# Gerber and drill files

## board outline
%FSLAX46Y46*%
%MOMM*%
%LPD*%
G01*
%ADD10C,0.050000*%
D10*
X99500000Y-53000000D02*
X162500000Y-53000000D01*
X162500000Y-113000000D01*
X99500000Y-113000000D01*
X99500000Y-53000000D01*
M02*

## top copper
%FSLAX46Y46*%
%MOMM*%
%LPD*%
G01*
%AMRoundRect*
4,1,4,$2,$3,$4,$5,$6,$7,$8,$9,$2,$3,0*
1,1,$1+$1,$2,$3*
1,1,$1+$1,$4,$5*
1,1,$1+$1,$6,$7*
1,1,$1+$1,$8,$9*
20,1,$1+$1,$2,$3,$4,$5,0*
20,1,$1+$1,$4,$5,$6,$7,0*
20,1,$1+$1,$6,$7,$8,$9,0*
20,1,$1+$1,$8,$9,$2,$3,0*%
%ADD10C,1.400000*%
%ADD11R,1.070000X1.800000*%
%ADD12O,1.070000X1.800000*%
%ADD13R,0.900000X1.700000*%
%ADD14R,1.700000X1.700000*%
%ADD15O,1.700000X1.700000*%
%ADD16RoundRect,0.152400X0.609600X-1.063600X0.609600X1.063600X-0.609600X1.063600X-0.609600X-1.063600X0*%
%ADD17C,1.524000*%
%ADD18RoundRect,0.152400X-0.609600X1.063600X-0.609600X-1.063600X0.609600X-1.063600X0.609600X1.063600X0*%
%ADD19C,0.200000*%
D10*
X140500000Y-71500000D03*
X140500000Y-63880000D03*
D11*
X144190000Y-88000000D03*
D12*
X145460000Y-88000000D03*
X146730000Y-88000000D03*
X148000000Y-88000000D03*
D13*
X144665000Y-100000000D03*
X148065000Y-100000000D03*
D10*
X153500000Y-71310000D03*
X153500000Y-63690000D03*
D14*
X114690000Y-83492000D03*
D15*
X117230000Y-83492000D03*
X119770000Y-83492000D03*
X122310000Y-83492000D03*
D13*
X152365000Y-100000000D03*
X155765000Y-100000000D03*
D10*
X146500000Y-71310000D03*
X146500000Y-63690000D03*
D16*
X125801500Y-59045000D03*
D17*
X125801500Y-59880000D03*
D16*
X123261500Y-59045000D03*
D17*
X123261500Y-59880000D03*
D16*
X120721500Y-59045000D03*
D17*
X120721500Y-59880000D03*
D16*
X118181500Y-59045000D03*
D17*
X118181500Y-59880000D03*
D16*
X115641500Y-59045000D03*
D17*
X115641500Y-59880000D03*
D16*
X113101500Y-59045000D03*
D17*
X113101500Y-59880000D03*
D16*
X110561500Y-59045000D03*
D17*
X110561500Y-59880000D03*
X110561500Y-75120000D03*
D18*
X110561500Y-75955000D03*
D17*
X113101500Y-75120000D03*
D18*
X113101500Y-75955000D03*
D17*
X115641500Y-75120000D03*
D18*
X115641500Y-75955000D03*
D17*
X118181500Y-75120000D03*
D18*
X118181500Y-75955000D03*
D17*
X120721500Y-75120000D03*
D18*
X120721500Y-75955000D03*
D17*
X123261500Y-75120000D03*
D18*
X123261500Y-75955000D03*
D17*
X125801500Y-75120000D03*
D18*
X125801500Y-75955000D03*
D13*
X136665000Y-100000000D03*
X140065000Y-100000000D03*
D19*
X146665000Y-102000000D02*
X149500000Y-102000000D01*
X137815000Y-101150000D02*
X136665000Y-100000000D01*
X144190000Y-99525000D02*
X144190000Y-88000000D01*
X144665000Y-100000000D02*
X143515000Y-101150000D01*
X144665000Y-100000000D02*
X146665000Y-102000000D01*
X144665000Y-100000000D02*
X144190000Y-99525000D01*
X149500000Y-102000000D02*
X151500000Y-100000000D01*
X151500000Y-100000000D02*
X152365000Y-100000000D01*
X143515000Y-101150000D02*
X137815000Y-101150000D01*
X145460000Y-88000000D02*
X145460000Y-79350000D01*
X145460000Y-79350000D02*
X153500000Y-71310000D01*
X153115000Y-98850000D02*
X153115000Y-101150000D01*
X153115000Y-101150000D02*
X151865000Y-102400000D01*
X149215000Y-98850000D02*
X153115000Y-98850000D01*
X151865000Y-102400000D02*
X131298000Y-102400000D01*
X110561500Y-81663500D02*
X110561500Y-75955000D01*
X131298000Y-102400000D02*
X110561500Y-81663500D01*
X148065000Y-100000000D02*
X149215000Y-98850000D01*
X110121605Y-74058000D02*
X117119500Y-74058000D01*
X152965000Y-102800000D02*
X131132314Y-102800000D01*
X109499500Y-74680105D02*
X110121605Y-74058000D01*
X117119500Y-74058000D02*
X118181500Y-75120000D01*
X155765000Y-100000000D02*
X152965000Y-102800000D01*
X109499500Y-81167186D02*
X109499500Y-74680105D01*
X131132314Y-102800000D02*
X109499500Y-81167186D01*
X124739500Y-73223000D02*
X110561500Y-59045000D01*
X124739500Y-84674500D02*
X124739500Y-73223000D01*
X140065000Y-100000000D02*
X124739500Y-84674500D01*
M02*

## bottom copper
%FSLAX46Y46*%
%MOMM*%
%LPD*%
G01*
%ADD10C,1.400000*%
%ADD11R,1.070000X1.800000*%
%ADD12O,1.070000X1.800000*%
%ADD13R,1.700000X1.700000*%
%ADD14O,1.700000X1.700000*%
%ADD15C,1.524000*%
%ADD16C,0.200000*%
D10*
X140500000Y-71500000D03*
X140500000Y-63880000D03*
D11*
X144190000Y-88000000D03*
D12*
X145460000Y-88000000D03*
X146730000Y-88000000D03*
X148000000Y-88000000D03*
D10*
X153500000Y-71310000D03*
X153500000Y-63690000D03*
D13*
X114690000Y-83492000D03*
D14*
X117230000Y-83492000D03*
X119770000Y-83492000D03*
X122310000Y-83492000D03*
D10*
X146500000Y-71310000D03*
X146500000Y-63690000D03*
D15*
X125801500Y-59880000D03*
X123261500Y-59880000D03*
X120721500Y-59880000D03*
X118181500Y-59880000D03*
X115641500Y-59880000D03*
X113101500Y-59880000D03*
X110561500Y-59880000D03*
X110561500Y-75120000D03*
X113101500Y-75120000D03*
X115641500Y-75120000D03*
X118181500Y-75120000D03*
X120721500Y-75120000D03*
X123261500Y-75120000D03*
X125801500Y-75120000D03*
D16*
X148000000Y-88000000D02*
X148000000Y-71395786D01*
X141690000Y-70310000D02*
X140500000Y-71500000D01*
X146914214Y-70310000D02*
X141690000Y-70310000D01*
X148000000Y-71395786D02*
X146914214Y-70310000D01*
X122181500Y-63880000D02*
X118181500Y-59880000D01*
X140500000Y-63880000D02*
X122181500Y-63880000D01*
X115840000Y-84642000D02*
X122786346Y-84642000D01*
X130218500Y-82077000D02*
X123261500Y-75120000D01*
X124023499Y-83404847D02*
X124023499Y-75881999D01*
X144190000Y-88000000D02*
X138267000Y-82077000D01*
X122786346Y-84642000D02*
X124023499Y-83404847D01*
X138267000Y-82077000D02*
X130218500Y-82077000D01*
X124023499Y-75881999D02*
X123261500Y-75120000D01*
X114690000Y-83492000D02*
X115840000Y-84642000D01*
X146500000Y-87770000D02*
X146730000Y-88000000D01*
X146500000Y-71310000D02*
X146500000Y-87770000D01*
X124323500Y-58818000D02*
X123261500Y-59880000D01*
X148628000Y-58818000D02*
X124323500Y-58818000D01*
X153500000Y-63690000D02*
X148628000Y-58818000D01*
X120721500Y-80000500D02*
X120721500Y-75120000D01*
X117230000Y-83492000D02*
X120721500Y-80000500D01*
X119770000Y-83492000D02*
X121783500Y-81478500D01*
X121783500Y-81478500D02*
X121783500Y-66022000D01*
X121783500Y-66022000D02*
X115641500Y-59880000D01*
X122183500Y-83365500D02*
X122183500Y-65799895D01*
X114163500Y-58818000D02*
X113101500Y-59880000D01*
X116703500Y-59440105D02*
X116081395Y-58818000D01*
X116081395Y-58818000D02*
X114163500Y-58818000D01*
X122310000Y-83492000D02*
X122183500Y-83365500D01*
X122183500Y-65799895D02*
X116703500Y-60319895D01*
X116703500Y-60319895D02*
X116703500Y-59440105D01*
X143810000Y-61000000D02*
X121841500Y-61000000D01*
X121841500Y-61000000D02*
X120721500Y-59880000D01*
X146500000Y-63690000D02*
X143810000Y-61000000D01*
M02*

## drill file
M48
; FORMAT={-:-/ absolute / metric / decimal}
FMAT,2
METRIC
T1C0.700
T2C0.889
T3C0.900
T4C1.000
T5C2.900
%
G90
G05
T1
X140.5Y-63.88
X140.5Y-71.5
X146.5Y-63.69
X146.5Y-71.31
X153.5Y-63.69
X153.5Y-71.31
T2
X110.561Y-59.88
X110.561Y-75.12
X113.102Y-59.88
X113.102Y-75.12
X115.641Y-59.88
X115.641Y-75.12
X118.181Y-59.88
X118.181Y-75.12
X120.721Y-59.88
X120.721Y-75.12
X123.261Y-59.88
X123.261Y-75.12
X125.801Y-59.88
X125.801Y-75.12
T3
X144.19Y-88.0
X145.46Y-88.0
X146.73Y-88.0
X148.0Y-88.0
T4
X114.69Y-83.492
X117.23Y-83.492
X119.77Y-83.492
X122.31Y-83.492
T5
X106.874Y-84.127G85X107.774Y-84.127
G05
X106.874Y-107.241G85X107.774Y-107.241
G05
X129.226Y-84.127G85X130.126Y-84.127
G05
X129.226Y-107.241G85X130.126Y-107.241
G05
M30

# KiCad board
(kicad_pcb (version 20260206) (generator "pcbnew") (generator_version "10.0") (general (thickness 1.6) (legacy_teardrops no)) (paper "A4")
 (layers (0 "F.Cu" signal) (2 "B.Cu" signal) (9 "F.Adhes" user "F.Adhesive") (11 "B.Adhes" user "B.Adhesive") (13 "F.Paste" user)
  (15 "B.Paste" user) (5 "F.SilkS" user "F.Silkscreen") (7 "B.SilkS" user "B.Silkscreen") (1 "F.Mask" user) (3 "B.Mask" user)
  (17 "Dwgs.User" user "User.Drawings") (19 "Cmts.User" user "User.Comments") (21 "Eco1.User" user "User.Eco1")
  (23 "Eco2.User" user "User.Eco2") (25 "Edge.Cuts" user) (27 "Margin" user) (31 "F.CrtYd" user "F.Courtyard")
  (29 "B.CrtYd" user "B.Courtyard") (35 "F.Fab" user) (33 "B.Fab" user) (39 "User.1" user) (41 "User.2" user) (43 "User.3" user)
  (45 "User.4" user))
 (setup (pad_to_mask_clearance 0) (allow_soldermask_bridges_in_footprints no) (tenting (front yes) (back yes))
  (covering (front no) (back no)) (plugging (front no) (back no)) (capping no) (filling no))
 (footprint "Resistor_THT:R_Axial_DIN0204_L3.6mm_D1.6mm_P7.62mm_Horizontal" (layer "F.Cu") (at 140.5 71.5 90)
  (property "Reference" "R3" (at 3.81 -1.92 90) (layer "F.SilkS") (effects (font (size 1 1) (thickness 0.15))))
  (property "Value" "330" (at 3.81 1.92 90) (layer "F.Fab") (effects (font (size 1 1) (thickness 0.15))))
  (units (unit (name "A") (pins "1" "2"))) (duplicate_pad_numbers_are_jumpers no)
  (pad "1" thru_hole circle (at 0 0 90) (size 1.4 1.4) (drill 0.7) (layers "*.Cu" "*.Mask") (remove_unused_layers no) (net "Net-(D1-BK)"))
  (pad "2" thru_hole circle (at 7.62 0 90) (size 1.4 1.4) (drill 0.7) (layers "*.Cu" "*.Mask") (remove_unused_layers no) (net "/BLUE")))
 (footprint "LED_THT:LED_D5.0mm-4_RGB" (layer "F.Cu") (at 144.19 88)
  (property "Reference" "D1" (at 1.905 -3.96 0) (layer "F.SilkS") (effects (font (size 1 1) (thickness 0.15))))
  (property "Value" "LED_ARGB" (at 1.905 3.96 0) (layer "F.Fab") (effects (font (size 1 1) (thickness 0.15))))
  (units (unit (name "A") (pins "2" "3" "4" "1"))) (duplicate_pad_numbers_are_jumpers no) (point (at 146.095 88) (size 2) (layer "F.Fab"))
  (pad "1" thru_hole rect (at 0 0) (size 1.07 1.8) (drill 0.9) (layers "*.Cu" "*.Mask") (remove_unused_layers no) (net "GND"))
  (pad "2" thru_hole oval (at 1.27 0) (size 1.07 1.8) (drill 0.9) (layers "*.Cu" "*.Mask") (remove_unused_layers no) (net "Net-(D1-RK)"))
  (pad "3" thru_hole oval (at 2.54 0) (size 1.07 1.8) (drill 0.9) (layers "*.Cu" "*.Mask") (remove_unused_layers no) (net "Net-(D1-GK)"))
  (pad "4" thru_hole oval (at 3.81 0) (size 1.07 1.8) (drill 0.9) (layers "*.Cu" "*.Mask") (remove_unused_layers no) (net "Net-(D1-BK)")))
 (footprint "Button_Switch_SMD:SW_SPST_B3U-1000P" (layer "F.Cu") (at 146.365 100)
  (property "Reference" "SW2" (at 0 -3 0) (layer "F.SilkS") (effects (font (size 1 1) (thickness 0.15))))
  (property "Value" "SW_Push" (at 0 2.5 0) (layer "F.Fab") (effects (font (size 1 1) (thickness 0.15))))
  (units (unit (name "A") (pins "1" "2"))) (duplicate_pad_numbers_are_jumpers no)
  (pad "1" smd rect (at -1.7 0) (size 0.9 1.7) (layers "F.Cu" "F.Mask" "F.Paste") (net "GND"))
  (pad "2" smd rect (at 1.7 0) (size 0.9 1.7) (layers "F.Cu" "F.Mask" "F.Paste") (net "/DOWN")))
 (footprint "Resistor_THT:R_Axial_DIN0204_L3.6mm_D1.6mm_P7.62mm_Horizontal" (layer "F.Cu") (at 153.5 71.31 90)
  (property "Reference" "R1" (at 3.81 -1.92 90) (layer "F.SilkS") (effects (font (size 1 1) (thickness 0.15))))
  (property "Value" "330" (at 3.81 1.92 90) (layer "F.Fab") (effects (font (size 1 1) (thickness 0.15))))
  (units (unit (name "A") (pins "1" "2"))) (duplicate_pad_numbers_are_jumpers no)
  (pad "1" thru_hole circle (at 0 0 90) (size 1.4 1.4) (drill 0.7) (layers "*.Cu" "*.Mask") (remove_unused_layers no) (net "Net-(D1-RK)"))
  (pad "2" thru_hole circle (at 7.62 0 90) (size 1.4 1.4) (drill 0.7) (layers "*.Cu" "*.Mask") (remove_unused_layers no) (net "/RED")))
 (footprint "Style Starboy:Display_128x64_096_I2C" (layer "F.Cu") (at 118.5 83.492)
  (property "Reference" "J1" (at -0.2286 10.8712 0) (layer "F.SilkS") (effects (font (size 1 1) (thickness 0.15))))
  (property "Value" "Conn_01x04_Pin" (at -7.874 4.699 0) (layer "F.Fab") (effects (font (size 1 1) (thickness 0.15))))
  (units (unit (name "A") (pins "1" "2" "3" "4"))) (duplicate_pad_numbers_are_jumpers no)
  (pad "" np_thru_hole oval (at -11.176 0.635) (size 3.8 2.9) (drill oval 3.8 2.9) (layers "*.Cu" "*.Mask"))
  (pad "" np_thru_hole oval (at -11.176 23.749) (size 3.8 2.9) (drill oval 3.8 2.9) (layers "*.Cu" "*.Mask"))
  (pad "" np_thru_hole oval (at 11.176 0.635) (size 3.8 2.9) (drill oval 3.8 2.9) (layers "*.Cu" "*.Mask"))
  (pad "" np_thru_hole oval (at 11.176 23.749) (size 3.8 2.9) (drill oval 3.8 2.9) (layers "*.Cu" "*.Mask"))
  (pad "1" thru_hole rect (at -3.81 0 90) (size 1.7 1.7) (drill 1) (layers "*.Cu" "*.Mask") (remove_unused_layers no) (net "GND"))
  (pad "2" thru_hole oval (at -1.27 0 90) (size 1.7 1.7) (drill 1) (layers "*.Cu" "*.Mask") (remove_unused_layers no) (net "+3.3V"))
  (pad "3" thru_hole oval (at 1.27 0 90) (size 1.7 1.7) (drill 1) (layers "*.Cu" "*.Mask") (remove_unused_layers no) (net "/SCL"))
  (pad "4" thru_hole oval (at 3.81 0 90) (size 1.7 1.7) (drill 1) (layers "*.Cu" "*.Mask") (remove_unused_layers no) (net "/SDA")))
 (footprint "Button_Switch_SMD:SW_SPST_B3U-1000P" (layer "F.Cu") (at 154.065 100)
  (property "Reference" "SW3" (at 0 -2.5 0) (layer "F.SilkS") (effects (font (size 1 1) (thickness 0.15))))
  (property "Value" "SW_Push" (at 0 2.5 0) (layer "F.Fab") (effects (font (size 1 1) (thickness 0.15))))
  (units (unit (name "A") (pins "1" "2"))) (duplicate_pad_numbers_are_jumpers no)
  (pad "1" smd rect (at -1.7 0) (size 0.9 1.7) (layers "F.Cu" "F.Mask" "F.Paste") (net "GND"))
  (pad "2" smd rect (at 1.7 0) (size 0.9 1.7) (layers "F.Cu" "F.Mask" "F.Paste") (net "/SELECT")))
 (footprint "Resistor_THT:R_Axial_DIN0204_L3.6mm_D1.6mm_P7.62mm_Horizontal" (layer "F.Cu") (at 146.5 71.31 90)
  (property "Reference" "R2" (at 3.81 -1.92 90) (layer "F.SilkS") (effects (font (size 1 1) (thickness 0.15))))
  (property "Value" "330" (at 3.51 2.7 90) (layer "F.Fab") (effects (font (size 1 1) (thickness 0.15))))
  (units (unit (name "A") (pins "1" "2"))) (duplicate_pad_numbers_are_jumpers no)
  (pad "1" thru_hole circle (at 0 0 90) (size 1.4 1.4) (drill 0.7) (layers "*.Cu" "*.Mask") (remove_unused_layers no) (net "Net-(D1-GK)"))
  (pad "2" thru_hole circle (at 7.62 0 90) (size 1.4 1.4) (drill 0.7) (layers "*.Cu" "*.Mask") (remove_unused_layers no) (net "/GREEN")))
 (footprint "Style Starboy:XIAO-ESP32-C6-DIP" (layer "F.Cu") (at 118.1815 67.5)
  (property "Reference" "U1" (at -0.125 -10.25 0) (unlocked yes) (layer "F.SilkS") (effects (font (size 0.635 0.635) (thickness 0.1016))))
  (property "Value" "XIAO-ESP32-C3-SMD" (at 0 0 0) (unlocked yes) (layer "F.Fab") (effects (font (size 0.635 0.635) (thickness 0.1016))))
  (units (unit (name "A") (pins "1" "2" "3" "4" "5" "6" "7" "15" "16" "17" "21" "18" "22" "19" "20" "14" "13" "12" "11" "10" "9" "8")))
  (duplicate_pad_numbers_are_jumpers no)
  (pad "1" smd roundrect (at 7.62 -8.455 90) (size 2.432 1.524) (layers "F.Cu" "F.Mask") (roundrect_rratio 0.1)
   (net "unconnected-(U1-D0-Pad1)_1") (thermal_bridge_angle 45))
  (pad "1" thru_hole circle (at 7.62 -7.62 90) (size 1.524 1.524) (drill 0.889) (layers "*.Cu" "*.Mask") (remove_unused_layers no)
   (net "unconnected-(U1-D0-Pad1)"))
  (pad "2" smd roundrect (at 5.08 -8.455 90) (size 2.432 1.524) (layers "F.Cu" "F.Mask") (roundrect_rratio 0.1) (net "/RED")
   (thermal_bridge_angle 45))
  (pad "2" thru_hole circle (at 5.08 -7.62 90) (size 1.524 1.524) (drill 0.889) (layers "*.Cu" "*.Mask") (remove_unused_layers no)
   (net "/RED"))
  (pad "3" smd roundrect (at 2.54 -8.455 90) (size 2.432 1.524) (layers "F.Cu" "F.Mask") (roundrect_rratio 0.1) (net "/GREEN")
   (thermal_bridge_angle 45))
  (pad "3" thru_hole circle (at 2.54 -7.62 90) (size 1.524 1.524) (drill 0.889) (layers "*.Cu" "*.Mask") (remove_unused_layers no)
   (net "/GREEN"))
  (pad "4" smd roundrect (at 0 -8.455 90) (size 2.432 1.524) (layers "F.Cu" "F.Mask") (roundrect_rratio 0.1) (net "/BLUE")
   (thermal_bridge_angle 45))
  (pad "4" thru_hole circle (at 0 -7.62 90) (size 1.524 1.524) (drill 0.889) (layers "*.Cu" "*.Mask") (remove_unused_layers no)
   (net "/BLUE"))
  (pad "5" smd roundrect (at -2.54 -8.455 90) (size 2.432 1.524) (layers "F.Cu" "F.Mask") (roundrect_rratio 0.1) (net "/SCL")
   (thermal_bridge_angle 45))
  (pad "5" thru_hole circle (at -2.54 -7.62 90) (size 1.524 1.524) (drill 0.889) (layers "*.Cu" "*.Mask") (remove_unused_layers no)
   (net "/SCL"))
  (pad "6" smd roundrect (at -5.08 -8.455 90) (size 2.432 1.524) (layers "F.Cu" "F.Mask") (roundrect_rratio 0.1) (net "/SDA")
   (thermal_bridge_angle 45))
  (pad "6" thru_hole circle (at -5.08 -7.62 90) (size 1.524 1.524) (drill 0.889) (layers "*.Cu" "*.Mask") (remove_unused_layers no)
   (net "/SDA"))
  (pad "7" smd roundrect (at -7.62 -8.455 90) (size 2.432 1.524) (layers "F.Cu" "F.Mask") (roundrect_rratio 0.1) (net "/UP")
   (thermal_bridge_angle 45))
  (pad "7" thru_hole circle (at -7.62 -7.62 90) (size 1.524 1.524) (drill 0.889) (layers "*.Cu" "*.Mask") (remove_unused_layers no)
   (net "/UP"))
  (pad "8" thru_hole circle (at -7.62 7.62 270) (size 1.524 1.524) (drill 0.889) (layers "*.Cu" "*.Mask") (remove_unused_layers no)
   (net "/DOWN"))
  (pad "8" smd roundrect (at -7.62 8.455 270) (size 2.432 1.524) (layers "F.Cu" "F.Mask") (roundrect_rratio 0.1) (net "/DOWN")
   (thermal_bridge_angle 45))
  (pad "9" thru_hole circle (at -5.08 7.62 270) (size 1.524 1.524) (drill 0.889) (layers "*.Cu" "*.Mask") (remove_unused_layers no)
   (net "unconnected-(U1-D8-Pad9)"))
  (pad "9" smd roundrect (at -5.08 8.455 270) (size 2.432 1.524) (layers "F.Cu" "F.Mask") (roundrect_rratio 0.1)
   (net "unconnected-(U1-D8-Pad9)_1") (thermal_bridge_angle 45))
  (pad "10" thru_hole circle (at -2.54 7.62 270) (size 1.524 1.524) (drill 0.889) (layers "*.Cu" "*.Mask") (remove_unused_layers no)
   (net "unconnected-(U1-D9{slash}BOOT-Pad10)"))
  (pad "10" smd roundrect (at -2.54 8.455 270) (size 2.432 1.524) (layers "F.Cu" "F.Mask") (roundrect_rratio 0.1)
   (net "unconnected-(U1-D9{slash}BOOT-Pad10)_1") (thermal_bridge_angle 45))
  (pad "11" thru_hole circle (at 0 7.62 270) (size 1.524 1.524) (drill 0.889) (layers "*.Cu" "*.Mask") (remove_unused_layers no)
   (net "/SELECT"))
  (pad "11" smd roundrect (at 0 8.455 270) (size 2.432 1.524) (layers "F.Cu" "F.Mask") (roundrect_rratio 0.1) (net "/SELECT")
   (thermal_bridge_angle 45))
  (pad "12" thru_hole circle (at 2.54 7.62 270) (size 1.524 1.524) (drill 0.889) (layers "*.Cu" "*.Mask") (remove_unused_layers no)
   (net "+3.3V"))
  (pad "12" smd roundrect (at 2.54 8.455 270) (size 2.432 1.524) (layers "F.Cu" "F.Mask") (roundrect_rratio 0.1) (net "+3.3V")
   (thermal_bridge_angle 45))
  (pad "13" thru_hole circle (at 5.08 7.62 270) (size 1.524 1.524) (drill 0.889) (layers "*.Cu" "*.Mask") (remove_unused_layers no)
   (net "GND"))
  (pad "13" smd roundrect (at 5.08 8.455 270) (size 2.432 1.524) (layers "F.Cu" "F.Mask") (roundrect_rratio 0.1) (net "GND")
   (thermal_bridge_angle 45))
  (pad "14" thru_hole circle (at 7.62 7.62 270) (size 1.524 1.524) (drill 0.889) (layers "*.Cu" "*.Mask") (remove_unused_layers no)
   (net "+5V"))
  (pad "14" smd roundrect (at 7.62 8.455 270) (size 2.432 1.524) (layers "F.Cu" "F.Mask") (roundrect_rratio 0.1) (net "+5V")
   (thermal_bridge_angle 45)))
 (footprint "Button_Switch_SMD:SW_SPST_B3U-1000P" (layer "F.Cu") (at 138.365 100)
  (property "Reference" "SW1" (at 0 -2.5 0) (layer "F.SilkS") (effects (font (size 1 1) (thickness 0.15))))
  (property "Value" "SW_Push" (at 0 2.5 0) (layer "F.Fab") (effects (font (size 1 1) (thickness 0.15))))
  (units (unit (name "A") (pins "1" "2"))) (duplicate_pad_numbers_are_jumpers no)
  (pad "1" smd rect (at -1.7 0) (size 0.9 1.7) (layers "F.Cu" "F.Mask" "F.Paste") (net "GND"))
  (pad "2" smd rect (at 1.7 0) (size 0.9 1.7) (layers "F.Cu" "F.Mask" "F.Paste") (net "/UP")))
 (gr_rect (start 99.5 53) (end 162.5 113) (stroke (width 0.05) (type default)) (fill no) (layer "Edge.Cuts"))
 (segment (start 148 88) (end 148 71.395786) (width 0.2) (layer "B.Cu") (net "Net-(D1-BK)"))
 (segment (start 141.69 70.31) (end 140.5 71.5) (width 0.2) (layer "B.Cu") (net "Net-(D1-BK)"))
 (segment (start 146.914214 70.31) (end 141.69 70.31) (width 0.2) (layer "B.Cu") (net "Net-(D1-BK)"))
 (segment (start 148 71.395786) (end 146.914214 70.31) (width 0.2) (layer "B.Cu") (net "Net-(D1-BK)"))
 (segment (start 122.1815 63.88) (end 118.1815 59.88) (width 0.2) (layer "B.Cu") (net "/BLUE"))
 (segment (start 140.5 63.88) (end 122.1815 63.88) (width 0.2) (layer "B.Cu") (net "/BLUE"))
 (segment (start 146.665 102) (end 149.5 102) (width 0.2) (layer "F.Cu") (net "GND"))
 (segment (start 137.815 101.15) (end 136.665 100) (width 0.2) (layer "F.Cu") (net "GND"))
 (segment (start 144.19 99.525) (end 144.19 88) (width 0.2) (layer "F.Cu") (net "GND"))
 (segment (start 144.665 100) (end 143.515 101.15) (width 0.2) (layer "F.Cu") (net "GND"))
 (segment (start 144.665 100) (end 146.665 102) (width 0.2) (layer "F.Cu") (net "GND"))
 (segment (start 144.665 100) (end 144.19 99.525) (width 0.2) (layer "F.Cu") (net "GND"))
 (segment (start 149.5 102) (end 151.5 100) (width 0.2) (layer "F.Cu") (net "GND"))
 (segment (start 151.5 100) (end 152.365 100) (width 0.2) (layer "F.Cu") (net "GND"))
 (segment (start 143.515 101.15) (end 137.815 101.15) (width 0.2) (layer "F.Cu") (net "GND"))
 (segment (start 115.84 84.642) (end 122.786346 84.642) (width 0.2) (layer "B.Cu") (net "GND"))
 (segment (start 130.2185 82.077) (end 123.2615 75.12) (width 0.2) (layer "B.Cu") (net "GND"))
 (segment (start 124.023499 83.404847) (end 124.023499 75.881999) (width 0.2) (layer "B.Cu") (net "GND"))
 (segment (start 144.19 88) (end 138.267 82.077) (width 0.2) (layer "B.Cu") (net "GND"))
 (segment (start 122.786346 84.642) (end 124.023499 83.404847) (width 0.2) (layer "B.Cu") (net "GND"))
 (segment (start 138.267 82.077) (end 130.2185 82.077) (width 0.2) (layer "B.Cu") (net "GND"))
 (segment (start 124.023499 75.881999) (end 123.2615 75.12) (width 0.2) (layer "B.Cu") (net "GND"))
 (segment (start 114.69 83.492) (end 115.84 84.642) (width 0.2) (layer "B.Cu") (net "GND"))
 (segment (start 145.46 88) (end 145.46 79.35) (width 0.2) (layer "F.Cu") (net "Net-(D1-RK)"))
 (segment (start 145.46 79.35) (end 153.5 71.31) (width 0.2) (layer "F.Cu") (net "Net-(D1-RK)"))
 (segment (start 146.5 87.77) (end 146.73 88) (width 0.2) (layer "B.Cu") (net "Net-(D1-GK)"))
 (segment (start 146.5 71.31) (end 146.5 87.77) (width 0.2) (layer "B.Cu") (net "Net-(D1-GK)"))
 (segment (start 153.115 98.85) (end 153.115 101.15) (width 0.2) (layer "F.Cu") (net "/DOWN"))
 (segment (start 153.115 101.15) (end 151.865 102.4) (width 0.2) (layer "F.Cu") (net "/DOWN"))
 (segment (start 149.215 98.85) (end 153.115 98.85) (width 0.2) (layer "F.Cu") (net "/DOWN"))
 (segment (start 151.865 102.4) (end 131.298 102.4) (width 0.2) (layer "F.Cu") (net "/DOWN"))
 (segment (start 110.5615 81.6635) (end 110.5615 75.955) (width 0.2) (layer "F.Cu") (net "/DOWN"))
 (segment (start 131.298 102.4) (end 110.5615 81.6635) (width 0.2) (layer "F.Cu") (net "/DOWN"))
 (segment (start 148.065 100) (end 149.215 98.85) (width 0.2) (layer "F.Cu") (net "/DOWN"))
 (segment (start 124.3235 58.818) (end 123.2615 59.88) (width 0.2) (layer "B.Cu") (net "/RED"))
 (segment (start 148.628 58.818) (end 124.3235 58.818) (width 0.2) (layer "B.Cu") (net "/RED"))
 (segment (start 153.5 63.69) (end 148.628 58.818) (width 0.2) (layer "B.Cu") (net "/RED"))
 (segment (start 120.7215 80.0005) (end 120.7215 75.12) (width 0.2) (layer "B.Cu") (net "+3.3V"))
 (segment (start 117.23 83.492) (end 120.7215 80.0005) (width 0.2) (layer "B.Cu") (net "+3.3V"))
 (segment (start 119.77 83.492) (end 121.7835 81.4785) (width 0.2) (layer "B.Cu") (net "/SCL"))
 (segment (start 121.7835 81.4785) (end 121.7835 66.022) (width 0.2) (layer "B.Cu") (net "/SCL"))
 (segment (start 121.7835 66.022) (end 115.6415 59.88) (width 0.2) (layer "B.Cu") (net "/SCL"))
 (segment (start 122.1835 83.3655) (end 122.1835 65.799895) (width 0.2) (layer "B.Cu") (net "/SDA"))
 (segment (start 114.1635 58.818) (end 113.1015 59.88) (width 0.2) (layer "B.Cu") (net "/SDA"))
 (segment (start 116.7035 59.440105) (end 116.081395 58.818) (width 0.2) (layer "B.Cu") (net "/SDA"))
 (segment (start 116.081395 58.818) (end 114.1635 58.818) (width 0.2) (layer "B.Cu") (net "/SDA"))
 (segment (start 122.31 83.492) (end 122.1835 83.3655) (width 0.2) (layer "B.Cu") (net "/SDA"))
 (segment (start 122.1835 65.799895) (end 116.7035 60.319895) (width 0.2) (layer "B.Cu") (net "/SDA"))
 (segment (start 116.7035 60.319895) (end 116.7035 59.440105) (width 0.2) (layer "B.Cu") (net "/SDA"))
 (segment (start 110.121605 74.058) (end 117.1195 74.058) (width 0.2) (layer "F.Cu") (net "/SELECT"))
 (segment (start 152.965 102.8) (end 131.132314 102.8) (width 0.2) (layer "F.Cu") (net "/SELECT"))
 (segment (start 109.4995 74.680105) (end 110.121605 74.058) (width 0.2) (layer "F.Cu") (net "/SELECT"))
 (segment (start 117.1195 74.058) (end 118.1815 75.12) (width 0.2) (layer "F.Cu") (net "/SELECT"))
 (segment (start 155.765 100) (end 152.965 102.8) (width 0.2) (layer "F.Cu") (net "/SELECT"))
 (segment (start 109.4995 81.167186) (end 109.4995 74.680105) (width 0.2) (layer "F.Cu") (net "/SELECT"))
 (segment (start 131.132314 102.8) (end 109.4995 81.167186) (width 0.2) (layer "F.Cu") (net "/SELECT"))
 (segment (start 143.81 61) (end 121.8415 61) (width 0.2) (layer "B.Cu") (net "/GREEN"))
 (segment (start 121.8415 61) (end 120.7215 59.88) (width 0.2) (layer "B.Cu") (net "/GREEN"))
 (segment (start 146.5 63.69) (end 143.81 61) (width 0.2) (layer "B.Cu") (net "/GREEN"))
 (segment (start 124.7395 73.223) (end 110.5615 59.045) (width 0.2) (layer "F.Cu") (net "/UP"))
 (segment (start 124.7395 84.6745) (end 124.7395 73.223) (width 0.2) (layer "F.Cu") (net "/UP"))
 (segment (start 140.065 100) (end 124.7395 84.6745) (width 0.2) (layer "F.Cu") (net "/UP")))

